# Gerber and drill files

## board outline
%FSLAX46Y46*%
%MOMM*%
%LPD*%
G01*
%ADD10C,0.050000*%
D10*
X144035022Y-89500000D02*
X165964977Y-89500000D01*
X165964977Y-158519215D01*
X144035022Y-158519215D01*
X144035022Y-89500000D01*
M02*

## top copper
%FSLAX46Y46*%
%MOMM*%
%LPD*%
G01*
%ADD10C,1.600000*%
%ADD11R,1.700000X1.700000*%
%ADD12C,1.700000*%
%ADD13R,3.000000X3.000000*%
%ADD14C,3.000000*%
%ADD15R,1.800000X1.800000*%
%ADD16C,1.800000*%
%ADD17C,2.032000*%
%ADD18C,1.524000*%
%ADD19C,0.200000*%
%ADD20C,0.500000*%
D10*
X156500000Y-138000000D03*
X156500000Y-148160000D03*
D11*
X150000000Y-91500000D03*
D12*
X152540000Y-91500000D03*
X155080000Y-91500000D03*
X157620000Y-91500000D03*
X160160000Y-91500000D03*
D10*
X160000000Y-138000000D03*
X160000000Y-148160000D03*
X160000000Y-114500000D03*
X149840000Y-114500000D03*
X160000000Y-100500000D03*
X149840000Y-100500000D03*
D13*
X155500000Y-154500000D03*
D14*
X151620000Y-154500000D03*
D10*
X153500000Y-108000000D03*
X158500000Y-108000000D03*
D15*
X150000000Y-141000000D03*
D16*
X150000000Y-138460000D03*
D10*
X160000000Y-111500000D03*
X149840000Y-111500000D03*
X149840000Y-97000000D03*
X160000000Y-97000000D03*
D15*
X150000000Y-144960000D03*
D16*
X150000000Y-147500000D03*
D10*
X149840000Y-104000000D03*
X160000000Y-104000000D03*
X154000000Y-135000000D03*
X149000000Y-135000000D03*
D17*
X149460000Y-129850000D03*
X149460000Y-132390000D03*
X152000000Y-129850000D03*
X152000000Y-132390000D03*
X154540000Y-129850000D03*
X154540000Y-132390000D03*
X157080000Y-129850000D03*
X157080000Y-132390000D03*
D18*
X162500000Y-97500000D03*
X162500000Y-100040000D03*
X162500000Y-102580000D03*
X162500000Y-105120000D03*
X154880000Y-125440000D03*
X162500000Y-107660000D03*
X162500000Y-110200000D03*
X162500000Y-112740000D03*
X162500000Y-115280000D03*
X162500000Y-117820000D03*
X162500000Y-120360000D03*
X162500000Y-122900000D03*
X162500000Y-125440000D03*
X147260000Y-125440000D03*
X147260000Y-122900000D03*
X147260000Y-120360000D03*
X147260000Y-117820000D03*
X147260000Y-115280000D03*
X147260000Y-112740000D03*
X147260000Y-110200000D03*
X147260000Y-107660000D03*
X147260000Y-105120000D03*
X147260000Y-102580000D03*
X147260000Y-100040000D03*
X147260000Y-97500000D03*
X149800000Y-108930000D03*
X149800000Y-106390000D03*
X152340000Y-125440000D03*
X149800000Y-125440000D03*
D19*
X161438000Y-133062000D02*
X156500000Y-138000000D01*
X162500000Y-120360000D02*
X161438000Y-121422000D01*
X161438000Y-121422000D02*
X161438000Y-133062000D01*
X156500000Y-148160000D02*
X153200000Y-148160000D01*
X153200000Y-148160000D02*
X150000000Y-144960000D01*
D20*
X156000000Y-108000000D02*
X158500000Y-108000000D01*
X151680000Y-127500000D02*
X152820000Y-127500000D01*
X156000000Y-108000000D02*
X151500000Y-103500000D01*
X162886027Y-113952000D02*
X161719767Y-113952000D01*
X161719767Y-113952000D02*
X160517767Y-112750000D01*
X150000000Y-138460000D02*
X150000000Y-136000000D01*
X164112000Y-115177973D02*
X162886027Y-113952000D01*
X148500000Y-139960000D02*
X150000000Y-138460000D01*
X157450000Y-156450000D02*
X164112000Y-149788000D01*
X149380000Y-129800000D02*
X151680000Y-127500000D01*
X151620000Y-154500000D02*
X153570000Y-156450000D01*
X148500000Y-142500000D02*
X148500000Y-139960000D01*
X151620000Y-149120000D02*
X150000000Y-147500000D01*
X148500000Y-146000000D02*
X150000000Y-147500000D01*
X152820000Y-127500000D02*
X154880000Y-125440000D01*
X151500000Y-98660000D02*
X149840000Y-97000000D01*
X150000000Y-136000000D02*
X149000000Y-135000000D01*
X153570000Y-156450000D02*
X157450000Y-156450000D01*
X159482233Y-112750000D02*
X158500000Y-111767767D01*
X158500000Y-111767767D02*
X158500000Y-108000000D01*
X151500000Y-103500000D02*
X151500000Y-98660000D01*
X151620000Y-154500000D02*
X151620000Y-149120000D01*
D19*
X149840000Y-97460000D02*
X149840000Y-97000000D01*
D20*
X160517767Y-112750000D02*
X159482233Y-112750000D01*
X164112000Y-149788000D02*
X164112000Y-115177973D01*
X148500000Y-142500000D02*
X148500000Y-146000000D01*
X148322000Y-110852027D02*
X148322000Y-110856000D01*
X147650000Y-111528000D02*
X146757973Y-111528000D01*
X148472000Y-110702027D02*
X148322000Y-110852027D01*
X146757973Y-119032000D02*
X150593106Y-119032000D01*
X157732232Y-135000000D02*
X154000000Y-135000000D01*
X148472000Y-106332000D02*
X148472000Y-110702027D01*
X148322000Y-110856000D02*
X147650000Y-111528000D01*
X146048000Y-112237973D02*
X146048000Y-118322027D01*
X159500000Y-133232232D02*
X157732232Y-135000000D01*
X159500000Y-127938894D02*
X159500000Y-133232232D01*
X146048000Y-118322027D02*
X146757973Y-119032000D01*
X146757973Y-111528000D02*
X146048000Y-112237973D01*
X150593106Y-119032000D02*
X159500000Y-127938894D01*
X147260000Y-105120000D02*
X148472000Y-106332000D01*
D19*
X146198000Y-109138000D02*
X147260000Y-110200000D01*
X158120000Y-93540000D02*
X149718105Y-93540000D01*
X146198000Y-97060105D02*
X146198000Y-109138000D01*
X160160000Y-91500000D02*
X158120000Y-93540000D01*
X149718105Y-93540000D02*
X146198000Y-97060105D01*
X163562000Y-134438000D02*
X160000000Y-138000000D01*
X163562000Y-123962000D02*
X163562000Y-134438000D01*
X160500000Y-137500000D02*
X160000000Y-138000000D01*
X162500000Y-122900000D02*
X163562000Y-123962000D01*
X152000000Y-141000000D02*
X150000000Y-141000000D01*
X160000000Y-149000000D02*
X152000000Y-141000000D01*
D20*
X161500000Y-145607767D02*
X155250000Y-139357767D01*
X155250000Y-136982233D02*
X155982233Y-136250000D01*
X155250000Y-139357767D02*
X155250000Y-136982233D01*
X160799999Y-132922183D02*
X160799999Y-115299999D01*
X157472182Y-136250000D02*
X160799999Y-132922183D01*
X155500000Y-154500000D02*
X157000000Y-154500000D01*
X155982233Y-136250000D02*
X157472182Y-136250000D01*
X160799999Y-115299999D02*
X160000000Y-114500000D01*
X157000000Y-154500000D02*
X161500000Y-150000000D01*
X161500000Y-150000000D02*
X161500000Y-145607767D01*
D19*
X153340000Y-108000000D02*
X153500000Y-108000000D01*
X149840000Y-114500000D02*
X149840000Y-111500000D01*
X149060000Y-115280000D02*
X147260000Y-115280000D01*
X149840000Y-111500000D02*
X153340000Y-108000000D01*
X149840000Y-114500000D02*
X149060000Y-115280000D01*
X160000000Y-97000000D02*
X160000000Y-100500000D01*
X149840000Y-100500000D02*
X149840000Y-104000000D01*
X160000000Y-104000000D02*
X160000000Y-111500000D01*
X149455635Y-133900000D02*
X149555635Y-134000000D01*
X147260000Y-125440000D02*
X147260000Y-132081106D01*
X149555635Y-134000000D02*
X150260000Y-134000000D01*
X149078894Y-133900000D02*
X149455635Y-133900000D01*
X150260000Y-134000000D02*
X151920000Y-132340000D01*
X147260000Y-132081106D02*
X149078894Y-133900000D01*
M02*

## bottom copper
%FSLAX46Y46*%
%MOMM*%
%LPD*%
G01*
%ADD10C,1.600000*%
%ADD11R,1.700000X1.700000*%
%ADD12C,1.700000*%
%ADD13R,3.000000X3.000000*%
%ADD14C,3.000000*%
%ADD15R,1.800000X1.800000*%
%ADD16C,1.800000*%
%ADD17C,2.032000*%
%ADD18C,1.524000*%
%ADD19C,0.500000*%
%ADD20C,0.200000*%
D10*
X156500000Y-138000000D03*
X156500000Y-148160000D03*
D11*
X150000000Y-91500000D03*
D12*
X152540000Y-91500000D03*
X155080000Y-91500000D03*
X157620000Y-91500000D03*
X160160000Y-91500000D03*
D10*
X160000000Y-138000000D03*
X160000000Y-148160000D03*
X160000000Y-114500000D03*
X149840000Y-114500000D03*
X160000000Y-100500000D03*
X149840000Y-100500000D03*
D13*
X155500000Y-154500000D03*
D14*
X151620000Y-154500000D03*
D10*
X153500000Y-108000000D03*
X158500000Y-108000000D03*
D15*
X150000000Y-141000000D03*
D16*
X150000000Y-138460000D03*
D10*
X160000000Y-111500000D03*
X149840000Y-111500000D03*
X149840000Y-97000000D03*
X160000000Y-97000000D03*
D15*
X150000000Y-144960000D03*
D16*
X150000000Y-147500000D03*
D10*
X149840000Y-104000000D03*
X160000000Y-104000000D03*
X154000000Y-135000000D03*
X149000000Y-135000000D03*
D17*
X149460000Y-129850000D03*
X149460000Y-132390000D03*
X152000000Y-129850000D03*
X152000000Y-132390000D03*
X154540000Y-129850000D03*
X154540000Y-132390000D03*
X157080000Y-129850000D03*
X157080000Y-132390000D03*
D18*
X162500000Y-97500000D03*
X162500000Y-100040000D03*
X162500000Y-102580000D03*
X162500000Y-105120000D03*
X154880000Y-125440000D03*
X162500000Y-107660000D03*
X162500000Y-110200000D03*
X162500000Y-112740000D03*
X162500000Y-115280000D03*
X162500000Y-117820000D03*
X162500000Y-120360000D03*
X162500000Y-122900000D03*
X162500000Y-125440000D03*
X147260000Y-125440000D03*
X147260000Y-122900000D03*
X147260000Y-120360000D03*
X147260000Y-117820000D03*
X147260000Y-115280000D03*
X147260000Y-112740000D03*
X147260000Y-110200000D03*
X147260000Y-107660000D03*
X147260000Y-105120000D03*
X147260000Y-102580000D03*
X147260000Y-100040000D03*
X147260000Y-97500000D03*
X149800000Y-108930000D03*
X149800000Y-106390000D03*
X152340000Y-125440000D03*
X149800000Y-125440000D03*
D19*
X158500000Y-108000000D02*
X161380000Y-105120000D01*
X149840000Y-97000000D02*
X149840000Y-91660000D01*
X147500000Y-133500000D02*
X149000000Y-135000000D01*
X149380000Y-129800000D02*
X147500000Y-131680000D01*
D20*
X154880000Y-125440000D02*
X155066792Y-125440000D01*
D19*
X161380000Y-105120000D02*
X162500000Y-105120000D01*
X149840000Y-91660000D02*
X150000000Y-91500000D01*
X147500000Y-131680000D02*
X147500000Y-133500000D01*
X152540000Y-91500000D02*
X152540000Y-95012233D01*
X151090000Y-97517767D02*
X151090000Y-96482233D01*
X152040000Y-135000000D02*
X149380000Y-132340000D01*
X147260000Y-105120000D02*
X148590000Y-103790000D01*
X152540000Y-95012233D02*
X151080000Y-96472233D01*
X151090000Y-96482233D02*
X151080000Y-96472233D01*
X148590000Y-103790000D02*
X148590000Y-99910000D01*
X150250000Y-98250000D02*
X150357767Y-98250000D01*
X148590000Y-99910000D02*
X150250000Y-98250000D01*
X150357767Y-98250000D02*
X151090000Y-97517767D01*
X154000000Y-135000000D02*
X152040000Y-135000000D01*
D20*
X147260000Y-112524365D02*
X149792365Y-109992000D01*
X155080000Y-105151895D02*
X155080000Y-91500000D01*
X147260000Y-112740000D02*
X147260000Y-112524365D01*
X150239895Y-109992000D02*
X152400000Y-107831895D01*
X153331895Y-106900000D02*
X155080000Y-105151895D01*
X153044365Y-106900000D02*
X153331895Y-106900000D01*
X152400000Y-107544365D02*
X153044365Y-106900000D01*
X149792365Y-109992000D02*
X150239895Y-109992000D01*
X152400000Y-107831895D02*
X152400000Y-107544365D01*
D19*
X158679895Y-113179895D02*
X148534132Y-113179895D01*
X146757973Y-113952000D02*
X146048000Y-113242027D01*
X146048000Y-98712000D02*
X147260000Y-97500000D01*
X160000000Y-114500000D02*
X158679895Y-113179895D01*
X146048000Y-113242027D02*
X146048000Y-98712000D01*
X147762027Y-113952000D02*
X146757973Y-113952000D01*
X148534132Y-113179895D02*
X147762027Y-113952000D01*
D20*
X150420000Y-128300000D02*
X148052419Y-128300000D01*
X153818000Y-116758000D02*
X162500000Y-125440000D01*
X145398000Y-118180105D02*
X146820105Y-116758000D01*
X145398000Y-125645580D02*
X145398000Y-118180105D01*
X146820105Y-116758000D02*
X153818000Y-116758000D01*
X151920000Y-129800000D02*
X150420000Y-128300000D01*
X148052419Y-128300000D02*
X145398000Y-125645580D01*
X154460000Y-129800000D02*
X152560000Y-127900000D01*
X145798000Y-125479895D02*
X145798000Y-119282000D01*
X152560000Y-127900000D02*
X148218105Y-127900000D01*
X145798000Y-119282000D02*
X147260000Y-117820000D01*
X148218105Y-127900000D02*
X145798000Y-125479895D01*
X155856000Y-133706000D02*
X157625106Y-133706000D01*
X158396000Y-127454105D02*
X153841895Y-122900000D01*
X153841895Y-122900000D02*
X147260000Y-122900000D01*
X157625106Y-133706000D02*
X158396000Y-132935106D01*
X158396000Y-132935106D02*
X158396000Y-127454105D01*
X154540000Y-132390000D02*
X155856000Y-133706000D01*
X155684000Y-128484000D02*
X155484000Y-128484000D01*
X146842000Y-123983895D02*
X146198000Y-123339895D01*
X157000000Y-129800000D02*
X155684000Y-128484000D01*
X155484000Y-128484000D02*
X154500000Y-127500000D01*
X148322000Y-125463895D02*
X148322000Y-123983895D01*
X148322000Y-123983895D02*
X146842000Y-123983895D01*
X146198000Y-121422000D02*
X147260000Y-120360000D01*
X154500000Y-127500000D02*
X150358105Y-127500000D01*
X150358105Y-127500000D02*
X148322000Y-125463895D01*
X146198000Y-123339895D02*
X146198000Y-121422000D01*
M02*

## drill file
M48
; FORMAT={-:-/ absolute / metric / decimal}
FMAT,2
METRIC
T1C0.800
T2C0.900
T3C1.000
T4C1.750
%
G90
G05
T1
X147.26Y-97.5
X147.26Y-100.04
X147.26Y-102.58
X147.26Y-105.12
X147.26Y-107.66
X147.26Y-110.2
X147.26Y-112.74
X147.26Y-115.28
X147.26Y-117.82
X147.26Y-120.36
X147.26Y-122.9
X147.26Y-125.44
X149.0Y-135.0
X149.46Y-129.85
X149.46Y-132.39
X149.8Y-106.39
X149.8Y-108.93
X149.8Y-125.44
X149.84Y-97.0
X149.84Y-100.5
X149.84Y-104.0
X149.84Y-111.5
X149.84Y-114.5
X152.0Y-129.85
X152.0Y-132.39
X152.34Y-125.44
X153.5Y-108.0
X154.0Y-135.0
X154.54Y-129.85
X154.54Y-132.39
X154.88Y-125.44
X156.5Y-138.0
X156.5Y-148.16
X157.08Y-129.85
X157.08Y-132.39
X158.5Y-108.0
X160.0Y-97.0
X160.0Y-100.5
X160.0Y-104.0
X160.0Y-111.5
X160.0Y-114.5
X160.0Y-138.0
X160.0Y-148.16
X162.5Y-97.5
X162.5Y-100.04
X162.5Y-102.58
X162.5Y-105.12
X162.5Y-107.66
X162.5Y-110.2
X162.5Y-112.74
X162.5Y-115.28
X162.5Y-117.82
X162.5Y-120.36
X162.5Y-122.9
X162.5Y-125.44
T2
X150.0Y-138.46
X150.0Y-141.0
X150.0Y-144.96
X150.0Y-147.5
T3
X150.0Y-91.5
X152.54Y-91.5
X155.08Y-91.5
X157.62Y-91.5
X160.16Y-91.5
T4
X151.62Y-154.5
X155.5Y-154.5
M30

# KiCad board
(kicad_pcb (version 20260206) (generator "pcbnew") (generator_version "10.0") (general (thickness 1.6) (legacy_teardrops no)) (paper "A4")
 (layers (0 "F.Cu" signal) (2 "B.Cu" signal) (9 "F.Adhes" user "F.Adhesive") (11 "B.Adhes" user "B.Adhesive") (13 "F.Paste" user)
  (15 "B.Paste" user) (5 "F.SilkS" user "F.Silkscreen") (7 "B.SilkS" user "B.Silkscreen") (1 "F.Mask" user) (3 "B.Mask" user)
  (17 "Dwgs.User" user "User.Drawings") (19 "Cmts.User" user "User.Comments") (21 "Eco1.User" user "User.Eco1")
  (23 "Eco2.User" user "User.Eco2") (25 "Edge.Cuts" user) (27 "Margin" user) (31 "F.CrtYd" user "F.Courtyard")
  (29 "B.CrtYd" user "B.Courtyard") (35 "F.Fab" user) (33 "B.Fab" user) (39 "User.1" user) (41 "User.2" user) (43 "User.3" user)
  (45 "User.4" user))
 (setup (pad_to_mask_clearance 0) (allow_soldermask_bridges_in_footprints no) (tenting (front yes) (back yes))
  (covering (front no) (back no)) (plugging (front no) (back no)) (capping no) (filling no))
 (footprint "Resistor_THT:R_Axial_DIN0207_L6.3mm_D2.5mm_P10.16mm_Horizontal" (layer "F.Cu") (at 156.5 138 -90)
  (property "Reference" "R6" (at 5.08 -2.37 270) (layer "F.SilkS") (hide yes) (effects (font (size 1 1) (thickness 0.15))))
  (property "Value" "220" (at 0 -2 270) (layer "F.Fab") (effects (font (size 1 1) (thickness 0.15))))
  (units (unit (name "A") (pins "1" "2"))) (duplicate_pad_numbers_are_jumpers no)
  (pad "1" thru_hole circle (at 0 0 270) (size 1.6 1.6) (drill 0.8) (layers "*.Cu" "*.Mask") (remove_unused_layers no) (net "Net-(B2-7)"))
  (pad "2" thru_hole circle (at 10.16 0 270) (size 1.6 1.6) (drill 0.8) (layers "*.Cu" "*.Mask") (remove_unused_layers no)
   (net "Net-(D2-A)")))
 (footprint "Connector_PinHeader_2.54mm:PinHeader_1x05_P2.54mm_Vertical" (layer "F.Cu") (at 150 91.5 90)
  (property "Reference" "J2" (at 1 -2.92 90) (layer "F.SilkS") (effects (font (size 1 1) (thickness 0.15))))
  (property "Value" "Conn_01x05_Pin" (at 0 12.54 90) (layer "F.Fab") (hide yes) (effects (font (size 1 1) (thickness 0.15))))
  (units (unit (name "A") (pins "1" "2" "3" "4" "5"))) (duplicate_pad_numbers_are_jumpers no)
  (pad "1" thru_hole rect (at 0 0 90) (size 1.7 1.7) (drill 1) (layers "*.Cu" "*.Mask") (remove_unused_layers no) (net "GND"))
  (pad "2" thru_hole circle (at 0 2.54 90) (size 1.7 1.7) (drill 1) (layers "*.Cu" "*.Mask") (remove_unused_layers no) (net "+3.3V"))
  (pad "3" thru_hole circle (at 0 5.08 90) (size 1.7 1.7) (drill 1) (layers "*.Cu" "*.Mask") (remove_unused_layers no) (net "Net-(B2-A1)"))
  (pad "4" thru_hole circle (at 0 7.62 90) (size 1.7 1.7) (drill 1) (layers "*.Cu" "*.Mask") (remove_unused_layers no)
   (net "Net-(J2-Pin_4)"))
  (pad "5" thru_hole circle (at 0 10.16 90) (size 1.7 1.7) (drill 1) (layers "*.Cu" "*.Mask") (remove_unused_layers no) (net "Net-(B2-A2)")))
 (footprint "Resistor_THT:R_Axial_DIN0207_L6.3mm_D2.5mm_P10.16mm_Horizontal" (layer "F.Cu") (at 160 138 -90)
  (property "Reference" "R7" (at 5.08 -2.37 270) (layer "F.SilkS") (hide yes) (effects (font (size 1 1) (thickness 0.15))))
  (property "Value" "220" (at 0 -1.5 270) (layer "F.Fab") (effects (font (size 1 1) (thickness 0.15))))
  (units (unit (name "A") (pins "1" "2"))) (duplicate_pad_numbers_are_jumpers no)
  (pad "1" thru_hole circle (at 0 0 270) (size 1.6 1.6) (drill 0.8) (layers "*.Cu" "*.Mask") (remove_unused_layers no) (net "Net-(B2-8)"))
  (pad "2" thru_hole circle (at 10.16 0 270) (size 1.6 1.6) (drill 0.8) (layers "*.Cu" "*.Mask") (remove_unused_layers no)
   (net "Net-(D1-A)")))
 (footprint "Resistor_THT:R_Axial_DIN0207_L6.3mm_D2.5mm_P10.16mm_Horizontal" (layer "F.Cu") (at 160 114.5 180)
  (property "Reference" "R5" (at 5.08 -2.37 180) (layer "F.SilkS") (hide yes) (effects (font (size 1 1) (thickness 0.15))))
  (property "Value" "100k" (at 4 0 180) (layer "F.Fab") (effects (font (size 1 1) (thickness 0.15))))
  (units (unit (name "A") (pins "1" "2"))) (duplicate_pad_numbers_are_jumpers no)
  (pad "1" thru_hole circle (at 0 0 180) (size 1.6 1.6) (drill 0.8) (layers "*.Cu" "*.Mask") (remove_unused_layers no) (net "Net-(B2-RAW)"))
  (pad "2" thru_hole circle (at 10.16 0 180) (size 1.6 1.6) (drill 0.8) (layers "*.Cu" "*.Mask") (remove_unused_layers no)
   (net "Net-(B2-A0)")))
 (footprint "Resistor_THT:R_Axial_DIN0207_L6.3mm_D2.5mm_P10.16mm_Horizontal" (layer "F.Cu") (at 160 100.5 180)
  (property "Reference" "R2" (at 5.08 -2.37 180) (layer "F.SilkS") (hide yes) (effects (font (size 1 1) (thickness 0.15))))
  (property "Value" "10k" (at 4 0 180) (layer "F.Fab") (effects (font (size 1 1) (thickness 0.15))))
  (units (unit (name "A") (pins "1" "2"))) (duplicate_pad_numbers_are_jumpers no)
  (pad "1" thru_hole circle (at 0 0 180) (size 1.6 1.6) (drill 0.8) (layers "*.Cu" "*.Mask") (remove_unused_layers no) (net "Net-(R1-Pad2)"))
  (pad "2" thru_hole circle (at 10.16 0 180) (size 1.6 1.6) (drill 0.8) (layers "*.Cu" "*.Mask") (remove_unused_layers no)
   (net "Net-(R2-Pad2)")))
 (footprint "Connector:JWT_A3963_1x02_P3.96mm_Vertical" (layer "F.Cu") (at 155.5 154.5 180)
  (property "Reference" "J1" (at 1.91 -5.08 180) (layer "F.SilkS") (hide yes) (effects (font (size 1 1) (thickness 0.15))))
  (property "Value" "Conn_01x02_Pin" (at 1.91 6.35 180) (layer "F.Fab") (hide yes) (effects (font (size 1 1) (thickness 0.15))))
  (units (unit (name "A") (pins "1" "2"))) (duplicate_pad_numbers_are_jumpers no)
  (pad "1" thru_hole rect (at 0 0 180) (size 3 3) (drill 1.75) (layers "*.Cu" "*.Mask") (remove_unused_layers no) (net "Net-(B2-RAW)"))
  (pad "2" thru_hole circle (at 3.88 0 180) (size 3 3) (drill 1.75) (layers "*.Cu" "*.Mask") (remove_unused_layers no) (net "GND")))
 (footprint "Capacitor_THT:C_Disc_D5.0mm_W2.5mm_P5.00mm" (layer "F.Cu") (at 153.5 108)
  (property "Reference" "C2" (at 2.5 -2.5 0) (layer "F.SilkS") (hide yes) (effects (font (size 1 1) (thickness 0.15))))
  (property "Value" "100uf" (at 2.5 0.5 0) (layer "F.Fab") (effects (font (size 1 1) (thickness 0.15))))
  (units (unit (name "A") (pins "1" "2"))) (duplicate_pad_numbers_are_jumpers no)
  (pad "1" thru_hole circle (at 0 0) (size 1.6 1.6) (drill 0.8) (layers "*.Cu" "*.Mask") (remove_unused_layers no) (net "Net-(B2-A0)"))
  (pad "2" thru_hole circle (at 5 0) (size 1.6 1.6) (drill 0.8) (layers "*.Cu" "*.Mask") (remove_unused_layers no) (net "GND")))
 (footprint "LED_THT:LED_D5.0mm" (layer "F.Cu") (at 150 141 90)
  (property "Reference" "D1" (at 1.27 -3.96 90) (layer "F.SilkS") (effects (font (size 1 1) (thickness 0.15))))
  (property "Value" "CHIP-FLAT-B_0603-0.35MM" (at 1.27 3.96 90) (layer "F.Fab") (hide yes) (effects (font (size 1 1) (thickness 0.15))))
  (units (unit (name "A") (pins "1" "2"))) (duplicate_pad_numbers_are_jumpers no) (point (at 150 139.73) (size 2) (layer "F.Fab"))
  (pad "1" thru_hole rect (at 0 0 90) (size 1.8 1.8) (drill 0.9) (layers "*.Cu" "*.Mask") (remove_unused_layers no) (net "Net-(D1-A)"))
  (pad "2" thru_hole circle (at 2.54 0 90) (size 1.8 1.8) (drill 0.9) (layers "*.Cu" "*.Mask") (remove_unused_layers no) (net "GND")))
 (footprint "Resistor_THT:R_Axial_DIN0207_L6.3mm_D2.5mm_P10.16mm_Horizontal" (layer "F.Cu") (at 160 111.5 180)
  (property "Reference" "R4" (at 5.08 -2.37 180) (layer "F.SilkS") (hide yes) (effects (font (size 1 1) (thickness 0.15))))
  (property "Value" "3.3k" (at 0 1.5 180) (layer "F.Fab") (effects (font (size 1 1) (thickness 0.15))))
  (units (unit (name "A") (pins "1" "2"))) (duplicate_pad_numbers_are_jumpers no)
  (pad "1" thru_hole circle (at 0 0 180) (size 1.6 1.6) (drill 0.8) (layers "*.Cu" "*.Mask") (remove_unused_layers no) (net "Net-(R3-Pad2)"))
  (pad "2" thru_hole circle (at 10.16 0 180) (size 1.6 1.6) (drill 0.8) (layers "*.Cu" "*.Mask") (remove_unused_layers no)
   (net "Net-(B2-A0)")))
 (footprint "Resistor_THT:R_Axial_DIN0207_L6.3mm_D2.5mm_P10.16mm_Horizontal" (layer "F.Cu") (at 149.84 97)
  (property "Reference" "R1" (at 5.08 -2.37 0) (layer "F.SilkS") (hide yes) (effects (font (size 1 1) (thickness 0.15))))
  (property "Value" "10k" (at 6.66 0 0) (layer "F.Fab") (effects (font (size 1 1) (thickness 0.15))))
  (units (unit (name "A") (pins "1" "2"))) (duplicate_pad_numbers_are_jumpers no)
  (pad "1" thru_hole circle (at 0 0) (size 1.6 1.6) (drill 0.8) (layers "*.Cu" "*.Mask") (remove_unused_layers no) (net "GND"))
  (pad "2" thru_hole circle (at 10.16 0) (size 1.6 1.6) (drill 0.8) (layers "*.Cu" "*.Mask") (remove_unused_layers no) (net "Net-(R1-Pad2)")))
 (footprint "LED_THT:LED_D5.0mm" (layer "F.Cu") (at 150 144.96 -90)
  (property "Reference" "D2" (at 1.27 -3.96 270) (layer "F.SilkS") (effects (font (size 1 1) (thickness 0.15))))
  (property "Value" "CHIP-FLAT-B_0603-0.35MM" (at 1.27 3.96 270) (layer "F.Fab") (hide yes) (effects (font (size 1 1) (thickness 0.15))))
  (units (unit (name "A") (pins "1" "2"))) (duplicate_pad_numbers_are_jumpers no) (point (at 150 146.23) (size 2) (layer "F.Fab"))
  (pad "1" thru_hole rect (at 0 0 270) (size 1.8 1.8) (drill 0.9) (layers "*.Cu" "*.Mask") (remove_unused_layers no) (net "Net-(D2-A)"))
  (pad "2" thru_hole circle (at 2.54 0 270) (size 1.8 1.8) (drill 0.9) (layers "*.Cu" "*.Mask") (remove_unused_layers no) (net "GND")))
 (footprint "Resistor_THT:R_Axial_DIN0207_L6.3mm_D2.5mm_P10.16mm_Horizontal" (layer "F.Cu") (at 149.84 104)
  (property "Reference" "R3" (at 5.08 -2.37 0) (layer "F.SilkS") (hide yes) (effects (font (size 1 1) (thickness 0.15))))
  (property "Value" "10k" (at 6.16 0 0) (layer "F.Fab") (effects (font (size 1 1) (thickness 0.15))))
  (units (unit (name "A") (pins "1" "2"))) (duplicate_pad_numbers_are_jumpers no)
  (pad "1" thru_hole circle (at 0 0) (size 1.6 1.6) (drill 0.8) (layers "*.Cu" "*.Mask") (remove_unused_layers no) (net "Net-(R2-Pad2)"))
  (pad "2" thru_hole circle (at 10.16 0) (size 1.6 1.6) (drill 0.8) (layers "*.Cu" "*.Mask") (remove_unused_layers no) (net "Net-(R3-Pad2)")))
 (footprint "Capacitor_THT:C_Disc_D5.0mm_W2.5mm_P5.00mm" (layer "F.Cu") (at 154 135 180)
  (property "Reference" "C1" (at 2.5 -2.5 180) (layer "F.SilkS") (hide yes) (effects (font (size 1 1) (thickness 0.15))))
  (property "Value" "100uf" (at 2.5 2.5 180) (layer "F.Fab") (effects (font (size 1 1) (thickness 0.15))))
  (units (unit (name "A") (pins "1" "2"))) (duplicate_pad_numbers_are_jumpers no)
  (pad "1" thru_hole circle (at 0 0 180) (size 1.6 1.6) (drill 0.8) (layers "*.Cu" "*.Mask") (remove_unused_layers no) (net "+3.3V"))
  (pad "2" thru_hole circle (at 5 0 180) (size 1.6 1.6) (drill 0.8) (layers "*.Cu" "*.Mask") (remove_unused_layers no) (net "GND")))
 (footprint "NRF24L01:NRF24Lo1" (layer "B.Cu") (at 155.175 142.55 -90)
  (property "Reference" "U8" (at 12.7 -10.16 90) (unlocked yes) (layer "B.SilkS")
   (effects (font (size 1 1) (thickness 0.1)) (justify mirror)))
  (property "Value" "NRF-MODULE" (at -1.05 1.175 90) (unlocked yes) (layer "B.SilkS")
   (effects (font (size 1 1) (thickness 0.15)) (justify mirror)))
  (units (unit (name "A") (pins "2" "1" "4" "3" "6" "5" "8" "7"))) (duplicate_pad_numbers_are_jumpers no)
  (pad "1" thru_hole circle (at -12.7 5.715 270) (size 2.032 2.032) (drill 0.8) (layers "*.Cu" "*.Mask") (remove_unused_layers no)
   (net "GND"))
  (pad "2" thru_hole circle (at -10.16 5.715 270) (size 2.032 2.032) (drill 0.8) (layers "*.Cu" "*.Mask") (remove_unused_layers no)
   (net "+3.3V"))
  (pad "3" thru_hole circle (at -12.7 3.175 270) (size 2.032 2.032) (drill 0.8) (layers "*.Cu" "*.Mask") (remove_unused_layers no)
   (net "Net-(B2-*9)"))
  (pad "4" thru_hole circle (at -10.16 3.175 270) (size 2.032 2.032) (drill 0.8) (layers "*.Cu" "*.Mask") (remove_unused_layers no)
   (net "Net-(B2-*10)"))
  (pad "5" thru_hole circle (at -12.7 0.635 270) (size 2.032 2.032) (drill 0.8) (layers "*.Cu" "*.Mask") (remove_unused_layers no)
   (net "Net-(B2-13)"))
  (pad "6" thru_hole circle (at -10.16 0.635 270) (size 2.032 2.032) (drill 0.8) (layers "*.Cu" "*.Mask") (remove_unused_layers no)
   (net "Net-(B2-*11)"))
  (pad "7" thru_hole circle (at -12.7 -1.905 270) (size 2.032 2.032) (drill 0.8) (layers "*.Cu" "*.Mask") (remove_unused_layers no)
   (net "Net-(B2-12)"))
  (pad "8" thru_hole circle (at -10.16 -1.905 270) (size 2.032 2.032) (drill 0.8) (layers "*.Cu" "*.Mask") (remove_unused_layers no)
   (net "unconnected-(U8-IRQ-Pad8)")))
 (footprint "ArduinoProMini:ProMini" (layer "B.Cu") (at 154.88 110.2 180)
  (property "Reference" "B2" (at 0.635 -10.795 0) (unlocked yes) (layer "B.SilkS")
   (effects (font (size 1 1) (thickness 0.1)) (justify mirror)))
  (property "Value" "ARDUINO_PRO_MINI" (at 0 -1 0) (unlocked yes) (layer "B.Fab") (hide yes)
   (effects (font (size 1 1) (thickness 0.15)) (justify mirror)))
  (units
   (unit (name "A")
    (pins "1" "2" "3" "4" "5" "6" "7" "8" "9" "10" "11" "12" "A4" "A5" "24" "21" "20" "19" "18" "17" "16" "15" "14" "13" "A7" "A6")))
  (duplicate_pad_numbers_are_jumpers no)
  (pad "1" thru_hole circle (at -7.62 12.7 180) (size 1.524 1.524) (drill 0.8) (layers "*.Cu" "*.Mask") (remove_unused_layers no)
   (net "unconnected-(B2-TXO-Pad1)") (thermal_bridge_angle 90))
  (pad "2" thru_hole circle (at -7.62 10.16 180) (size 1.524 1.524) (drill 0.8) (layers "*.Cu" "*.Mask") (remove_unused_layers no)
   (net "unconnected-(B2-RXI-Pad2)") (thermal_bridge_angle 90))
  (pad "3" thru_hole circle (at -7.62 7.62 180) (size 1.524 1.524) (drill 0.8) (layers "*.Cu" "*.Mask") (remove_unused_layers no)
   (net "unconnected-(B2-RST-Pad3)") (thermal_bridge_angle 90))
  (pad "4" thru_hole circle (at -7.62 5.08 180) (size 1.524 1.524) (drill 0.8) (layers "*.Cu" "*.Mask") (remove_unused_layers no)
   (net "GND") (thermal_bridge_angle 90))
  (pad "4" thru_hole circle (at 0 -15.24 180) (size 1.524 1.524) (drill 0.8) (layers "*.Cu" "*.Mask") (remove_unused_layers no) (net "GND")
   (thermal_bridge_angle 90))
  (pad "5" thru_hole circle (at -7.62 2.54 180) (size 1.524 1.524) (drill 0.8) (layers "*.Cu" "*.Mask") (remove_unused_layers no)
   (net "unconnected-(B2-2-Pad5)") (thermal_bridge_angle 90))
  (pad "6" thru_hole circle (at -7.62 0 180) (size 1.524 1.524) (drill 0.8) (layers "*.Cu" "*.Mask") (remove_unused_layers no)
   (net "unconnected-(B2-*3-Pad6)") (thermal_bridge_angle 90))
  (pad "7" thru_hole circle (at -7.62 -2.54 180) (size 1.524 1.524) (drill 0.8) (layers "*.Cu" "*.Mask") (remove_unused_layers no)
   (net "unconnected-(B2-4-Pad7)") (thermal_bridge_angle 90))
  (pad "8" thru_hole circle (at -7.62 -5.08 180) (size 1.524 1.524) (drill 0.8) (layers "*.Cu" "*.Mask") (remove_unused_layers no)
   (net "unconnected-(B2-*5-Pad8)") (thermal_bridge_angle 90))
  (pad "9" thru_hole circle (at -7.62 -7.62 180) (size 1.524 1.524) (drill 0.8) (layers "*.Cu" "*.Mask") (remove_unused_layers no)
   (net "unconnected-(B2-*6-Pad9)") (thermal_bridge_angle 90))
  (pad "10" thru_hole circle (at -7.62 -10.16 180) (size 1.524 1.524) (drill 0.8) (layers "*.Cu" "*.Mask") (remove_unused_layers no)
   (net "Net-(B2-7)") (thermal_bridge_angle 90))
  (pad "11" thru_hole circle (at -7.62 -12.7 180) (size 1.524 1.524) (drill 0.8) (layers "*.Cu" "*.Mask") (remove_unused_layers no)
   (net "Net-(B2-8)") (thermal_bridge_angle 90))
  (pad "12" thru_hole circle (at -7.62 -15.24 180) (size 1.524 1.524) (drill 0.8) (layers "*.Cu" "*.Mask") (remove_unused_layers no)
   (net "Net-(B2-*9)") (thermal_bridge_angle 90))
  (pad "13" thru_hole circle (at 7.62 -15.24 180) (size 1.524 1.524) (drill 0.8) (layers "*.Cu" "*.Mask") (remove_unused_layers no)
   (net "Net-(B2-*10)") (thermal_bridge_angle 90))
  (pad "14" thru_hole circle (at 7.62 -12.7 180) (size 1.524 1.524) (drill 0.8) (layers "*.Cu" "*.Mask") (remove_unused_layers no)
   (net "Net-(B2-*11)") (thermal_bridge_angle 90))
  (pad "15" thru_hole circle (at 7.62 -10.16 180) (size 1.524 1.524) (drill 0.8) (layers "*.Cu" "*.Mask") (remove_unused_layers no)
   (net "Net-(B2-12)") (thermal_bridge_angle 90))
  (pad "16" thru_hole circle (at 7.62 -7.62 180) (size 1.524 1.524) (drill 0.8) (layers "*.Cu" "*.Mask") (remove_unused_layers no)
   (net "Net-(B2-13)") (thermal_bridge_angle 90))
  (pad "17" thru_hole circle (at 7.62 -5.08 180) (size 1.524 1.524) (drill 0.8) (layers "*.Cu" "*.Mask") (remove_unused_layers no)
   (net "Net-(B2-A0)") (thermal_bridge_angle 90))
  (pad "18" thru_hole circle (at 7.62 -2.54 180) (size 1.524 1.524) (drill 0.8) (layers "*.Cu" "*.Mask") (remove_unused_layers no)
   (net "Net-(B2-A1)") (thermal_bridge_angle 90))
  (pad "19" thru_hole circle (at 7.62 0 180) (size 1.524 1.524) (drill 0.8) (layers "*.Cu" "*.Mask") (remove_unused_layers no)
   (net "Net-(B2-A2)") (thermal_bridge_angle 90))
  (pad "20" thru_hole circle (at 7.62 2.54 180) (size 1.524 1.524) (drill 0.8) (layers "*.Cu" "*.Mask") (remove_unused_layers no)
   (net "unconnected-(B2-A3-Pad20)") (thermal_bridge_angle 90))
  (pad "21" thru_hole circle (at 7.62 5.08 180) (size 1.524 1.524) (drill 0.8) (layers "*.Cu" "*.Mask") (remove_unused_layers no)
   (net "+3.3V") (thermal_bridge_angle 90))
  (pad "22" thru_hole circle (at 7.62 7.62 180) (size 1.524 1.524) (drill 0.8) (layers "*.Cu" "*.Mask") (remove_unused_layers no)
   (thermal_bridge_angle 90))
  (pad "23" thru_hole circle (at 7.62 10.16 180) (size 1.524 1.524) (drill 0.8) (layers "*.Cu" "*.Mask") (remove_unused_layers no)
   (thermal_bridge_angle 90))
  (pad "24" thru_hole circle (at 7.62 12.7 180) (size 1.524 1.524) (drill 0.8) (layers "*.Cu" "*.Mask") (remove_unused_layers no)
   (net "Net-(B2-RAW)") (thermal_bridge_angle 90))
  (pad "A4" thru_hole circle (at 5.08 1.27 180) (size 1.524 1.524) (drill 0.8) (layers "*.Cu" "*.Mask") (remove_unused_layers no)
   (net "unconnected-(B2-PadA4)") (thermal_bridge_angle 90))
  (pad "A5" thru_hole circle (at 5.08 3.81 180) (size 1.524 1.524) (drill 0.8) (layers "*.Cu" "*.Mask") (remove_unused_layers no)
   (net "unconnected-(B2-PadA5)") (thermal_bridge_angle 90))
  (pad "A6" thru_hole circle (at 2.54 -15.24 180) (size 1.524 1.524) (drill 0.8) (layers "*.Cu" "*.Mask") (remove_unused_layers no)
   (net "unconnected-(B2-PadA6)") (thermal_bridge_angle 90))
  (pad "A7" thru_hole circle (at 5.08 -15.24 180) (size 1.524 1.524) (drill 0.8) (layers "*.Cu" "*.Mask") (remove_unused_layers no)
   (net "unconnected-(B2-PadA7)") (thermal_bridge_angle 90)))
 (gr_rect (start 144.035022 89.5) (end 165.964977 158.519215) (stroke (width 0.05) (type default)) (fill no) (layer "Edge.Cuts"))
 (segment (start 161.438 133.062) (end 156.5 138) (width 0.2) (layer "F.Cu") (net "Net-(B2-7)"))
 (segment (start 162.5 120.36) (end 161.438 121.422) (width 0.2) (layer "F.Cu") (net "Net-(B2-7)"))
 (segment (start 161.438 121.422) (end 161.438 133.062) (width 0.2) (layer "F.Cu") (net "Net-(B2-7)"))
 (segment (start 156.5 148.16) (end 153.2 148.16) (width 0.2) (layer "F.Cu") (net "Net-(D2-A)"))
 (segment (start 153.2 148.16) (end 150 144.96) (width 0.2) (layer "F.Cu") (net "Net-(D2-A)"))
 (segment (start 156 108) (end 158.5 108) (width 0.5) (layer "F.Cu") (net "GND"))
 (segment (start 151.68 127.5) (end 152.82 127.5) (width 0.5) (layer "F.Cu") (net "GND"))
 (segment (start 156 108) (end 151.5 103.5) (width 0.5) (layer "F.Cu") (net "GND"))
 (segment (start 162.886027 113.952) (end 161.719767 113.952) (width 0.5) (layer "F.Cu") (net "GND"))
 (segment (start 161.719767 113.952) (end 160.517767 112.75) (width 0.5) (layer "F.Cu") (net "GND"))
 (segment (start 150 138.46) (end 150 136) (width 0.5) (layer "F.Cu") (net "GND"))
 (segment (start 164.112 115.177973) (end 162.886027 113.952) (width 0.5) (layer "F.Cu") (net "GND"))
 (segment (start 148.5 139.96) (end 150 138.46) (width 0.5) (layer "F.Cu") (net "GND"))
 (segment (start 157.45 156.45) (end 164.112 149.788) (width 0.5) (layer "F.Cu") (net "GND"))
 (segment (start 149.38 129.8) (end 151.68 127.5) (width 0.5) (layer "F.Cu") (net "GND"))
 (segment (start 151.62 154.5) (end 153.57 156.45) (width 0.5) (layer "F.Cu") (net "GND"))
 (segment (start 148.5 142.5) (end 148.5 139.96) (width 0.5) (layer "F.Cu") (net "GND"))
 (segment (start 151.62 149.12) (end 150 147.5) (width 0.5) (layer "F.Cu") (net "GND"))
 (segment (start 148.5 146) (end 150 147.5) (width 0.5) (layer "F.Cu") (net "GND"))
 (segment (start 152.82 127.5) (end 154.88 125.44) (width 0.5) (layer "F.Cu") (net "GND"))
 (segment (start 151.5 98.66) (end 149.84 97) (width 0.5) (layer "F.Cu") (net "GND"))
 (segment (start 150 136) (end 149 135) (width 0.5) (layer "F.Cu") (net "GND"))
 (segment (start 153.57 156.45) (end 157.45 156.45) (width 0.5) (layer "F.Cu") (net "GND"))
 (segment (start 159.482233 112.75) (end 158.5 111.767767) (width 0.5) (layer "F.Cu") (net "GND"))
 (segment (start 158.5 111.767767) (end 158.5 108) (width 0.5) (layer "F.Cu") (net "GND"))
 (segment (start 151.5 103.5) (end 151.5 98.66) (width 0.5) (layer "F.Cu") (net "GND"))
 (segment (start 151.62 154.5) (end 151.62 149.12) (width 0.5) (layer "F.Cu") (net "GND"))
 (segment (start 149.84 97.46) (end 149.84 97) (width 0.2) (layer "F.Cu") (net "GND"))
 (segment (start 160.517767 112.75) (end 159.482233 112.75) (width 0.5) (layer "F.Cu") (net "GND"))
 (segment (start 164.112 149.788) (end 164.112 115.177973) (width 0.5) (layer "F.Cu") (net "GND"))
 (segment (start 148.5 142.5) (end 148.5 146) (width 0.5) (layer "F.Cu") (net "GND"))
 (segment (start 158.5 108) (end 161.38 105.12) (width 0.5) (layer "B.Cu") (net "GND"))
 (segment (start 149.84 97) (end 149.84 91.66) (width 0.5) (layer "B.Cu") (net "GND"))
 (segment (start 147.5 133.5) (end 149 135) (width 0.5) (layer "B.Cu") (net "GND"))
 (segment (start 149.38 129.8) (end 147.5 131.68) (width 0.5) (layer "B.Cu") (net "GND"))
 (segment (start 154.88 125.44) (end 155.066792 125.44) (width 0.2) (layer "B.Cu") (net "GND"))
 (segment (start 161.38 105.12) (end 162.5 105.12) (width 0.5) (layer "B.Cu") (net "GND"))
 (segment (start 149.84 91.66) (end 150 91.5) (width 0.5) (layer "B.Cu") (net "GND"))
 (segment (start 147.5 131.68) (end 147.5 133.5) (width 0.5) (layer "B.Cu") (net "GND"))
 (segment (start 148.322 110.852027) (end 148.322 110.856) (width 0.5) (layer "F.Cu") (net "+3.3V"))
 (segment (start 147.65 111.528) (end 146.757973 111.528) (width 0.5) (layer "F.Cu") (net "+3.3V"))
 (segment (start 148.472 110.702027) (end 148.322 110.852027) (width 0.5) (layer "F.Cu") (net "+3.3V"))
 (segment (start 146.757973 119.032) (end 150.593106 119.032) (width 0.5) (layer "F.Cu") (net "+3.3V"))
 (segment (start 157.732232 135) (end 154 135) (width 0.5) (layer "F.Cu") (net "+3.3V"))
 (segment (start 148.472 106.332) (end 148.472 110.702027) (width 0.5) (layer "F.Cu") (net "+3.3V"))
 (segment (start 148.322 110.856) (end 147.65 111.528) (width 0.5) (layer "F.Cu") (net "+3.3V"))
 (segment (start 146.048 112.237973) (end 146.048 118.322027) (width 0.5) (layer "F.Cu") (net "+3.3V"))
 (segment (start 159.5 133.232232) (end 157.732232 135) (width 0.5) (layer "F.Cu") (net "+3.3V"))
 (segment (start 159.5 127.938894) (end 159.5 133.232232) (width 0.5) (layer "F.Cu") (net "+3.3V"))
 (segment (start 146.048 118.322027) (end 146.757973 119.032) (width 0.5) (layer "F.Cu") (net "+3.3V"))
 (segment (start 146.757973 111.528) (end 146.048 112.237973) (width 0.5) (layer "F.Cu") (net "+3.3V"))
 (segment (start 150.593106 119.032) (end 159.5 127.938894) (width 0.5) (layer "F.Cu") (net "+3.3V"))
 (segment (start 147.26 105.12) (end 148.472 106.332) (width 0.5) (layer "F.Cu") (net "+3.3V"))
 (segment (start 152.54 91.5) (end 152.54 95.012233) (width 0.5) (layer "B.Cu") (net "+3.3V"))
 (segment (start 151.09 97.517767) (end 151.09 96.482233) (width 0.5) (layer "B.Cu") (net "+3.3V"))
 (segment (start 152.04 135) (end 149.38 132.34) (width 0.5) (layer "B.Cu") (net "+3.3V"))
 (segment (start 147.26 105.12) (end 148.59 103.79) (width 0.5) (layer "B.Cu") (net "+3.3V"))
 (segment (start 152.54 95.012233) (end 151.08 96.472233) (width 0.5) (layer "B.Cu") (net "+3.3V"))
 (segment (start 151.09 96.482233) (end 151.08 96.472233) (width 0.5) (layer "B.Cu") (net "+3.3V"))
 (segment (start 148.59 103.79) (end 148.59 99.91) (width 0.5) (layer "B.Cu") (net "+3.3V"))
 (segment (start 150.25 98.25) (end 150.357767 98.25) (width 0.5) (layer "B.Cu") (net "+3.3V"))
 (segment (start 148.59 99.91) (end 150.25 98.25) (width 0.5) (layer "B.Cu") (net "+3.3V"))
 (segment (start 150.357767 98.25) (end 151.09 97.517767) (width 0.5) (layer "B.Cu") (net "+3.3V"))
 (segment (start 154 135) (end 152.04 135) (width 0.5) (layer "B.Cu") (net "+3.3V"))
 (segment (start 147.26 112.524365) (end 149.792365 109.992) (width 0.2) (layer "B.Cu") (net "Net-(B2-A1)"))
 (segment (start 155.08 105.151895) (end 155.08 91.5) (width 0.2) (layer "B.Cu") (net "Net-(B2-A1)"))
 (segment (start 147.26 112.74) (end 147.26 112.524365) (width 0.2) (layer "B.Cu") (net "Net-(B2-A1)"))
 (segment (start 150.239895 109.992) (end 152.4 107.831895) (width 0.2) (layer "B.Cu") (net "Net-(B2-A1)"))
 (segment (start 153.331895 106.9) (end 155.08 105.151895) (width 0.2) (layer "B.Cu") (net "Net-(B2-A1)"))
 (segment (start 153.044365 106.9) (end 153.331895 106.9) (width 0.2) (layer "B.Cu") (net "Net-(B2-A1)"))
 (segment (start 152.4 107.544365) (end 153.044365 106.9) (width 0.2) (layer "B.Cu") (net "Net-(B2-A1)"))
 (segment (start 149.792365 109.992) (end 150.239895 109.992) (width 0.2) (layer "B.Cu") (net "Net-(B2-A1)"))
 (segment (start 152.4 107.831895) (end 152.4 107.544365) (width 0.2) (layer "B.Cu") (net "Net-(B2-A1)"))
 (segment (start 146.198 109.138) (end 147.26 110.2) (width 0.2) (layer "F.Cu") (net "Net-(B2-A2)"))
 (segment (start 158.12 93.54) (end 149.718105 93.54) (width 0.2) (layer "F.Cu") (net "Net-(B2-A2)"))
 (segment (start 146.198 97.060105) (end 146.198 109.138) (width 0.2) (layer "F.Cu") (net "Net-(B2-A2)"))
 (segment (start 160.16 91.5) (end 158.12 93.54) (width 0.2) (layer "F.Cu") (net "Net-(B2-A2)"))
 (segment (start 149.718105 93.54) (end 146.198 97.060105) (width 0.2) (layer "F.Cu") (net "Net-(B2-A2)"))
 (segment (start 163.562 134.438) (end 160 138) (width 0.2) (layer "F.Cu") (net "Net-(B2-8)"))
 (segment (start 163.562 123.962) (end 163.562 134.438) (width 0.2) (layer "F.Cu") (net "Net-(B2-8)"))
 (segment (start 160.5 137.5) (end 160 138) (width 0.2) (layer "F.Cu") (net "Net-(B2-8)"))
 (segment (start 162.5 122.9) (end 163.562 123.962) (width 0.2) (layer "F.Cu") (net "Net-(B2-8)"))
 (segment (start 152 141) (end 150 141) (width 0.2) (layer "F.Cu") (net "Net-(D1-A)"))
 (segment (start 160 149) (end 152 141) (width 0.2) (layer "F.Cu") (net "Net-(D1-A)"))
 (segment (start 161.5 145.607767) (end 155.25 139.357767) (width 0.5) (layer "F.Cu") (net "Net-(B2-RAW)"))
 (segment (start 155.25 136.982233) (end 155.982233 136.25) (width 0.5) (layer "F.Cu") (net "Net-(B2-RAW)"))
 (segment (start 155.25 139.357767) (end 155.25 136.982233) (width 0.5) (layer "F.Cu") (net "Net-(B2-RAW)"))
 (segment (start 160.799999 132.922183) (end 160.799999 115.299999) (width 0.5) (layer "F.Cu") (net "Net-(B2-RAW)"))
 (segment (start 157.472182 136.25) (end 160.799999 132.922183) (width 0.5) (layer "F.Cu") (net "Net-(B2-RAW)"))
 (segment (start 155.5 154.5) (end 157 154.5) (width 0.5) (layer "F.Cu") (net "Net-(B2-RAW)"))
 (segment (start 155.982233 136.25) (end 157.472182 136.25) (width 0.5) (layer "F.Cu") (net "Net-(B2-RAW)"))
 (segment (start 160.799999 115.299999) (end 160 114.5) (width 0.5) (layer "F.Cu") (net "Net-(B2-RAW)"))
 (segment (start 157 154.5) (end 161.5 150) (width 0.5) (layer "F.Cu") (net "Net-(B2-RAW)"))
 (segment (start 161.5 150) (end 161.5 145.607767) (width 0.5) (layer "F.Cu") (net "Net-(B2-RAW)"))
 (segment (start 158.679895 113.179895) (end 148.534132 113.179895) (width 0.5) (layer "B.Cu") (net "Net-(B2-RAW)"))
 (segment (start 146.757973 113.952) (end 146.048 113.242027) (width 0.5) (layer "B.Cu") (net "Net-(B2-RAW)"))
 (segment (start 146.048 98.712) (end 147.26 97.5) (width 0.5) (layer "B.Cu") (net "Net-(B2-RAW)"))
 (segment (start 160 114.5) (end 158.679895 113.179895) (width 0.5) (layer "B.Cu") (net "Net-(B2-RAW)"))
 (segment (start 146.048 113.242027) (end 146.048 98.712) (width 0.5) (layer "B.Cu") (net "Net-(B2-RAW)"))
 (segment (start 147.762027 113.952) (end 146.757973 113.952) (width 0.5) (layer "B.Cu") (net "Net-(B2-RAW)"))
 (segment (start 148.534132 113.179895) (end 147.762027 113.952) (width 0.5) (layer "B.Cu") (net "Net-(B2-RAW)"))
 (segment (start 153.34 108) (end 153.5 108) (width 0.2) (layer "F.Cu") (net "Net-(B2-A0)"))
 (segment (start 149.84 114.5) (end 149.84 111.5) (width 0.2) (layer "F.Cu") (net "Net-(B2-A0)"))
 (segment (start 149.06 115.28) (end 147.26 115.28) (width 0.2) (layer "F.Cu") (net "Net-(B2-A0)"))
 (segment (start 149.84 111.5) (end 153.34 108) (width 0.2) (layer "F.Cu") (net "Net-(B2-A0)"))
 (segment (start 149.84 114.5) (end 149.06 115.28) (width 0.2) (layer "F.Cu") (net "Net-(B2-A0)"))
 (segment (start 160 97) (end 160 100.5) (width 0.2) (layer "F.Cu") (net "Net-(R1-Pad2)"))
 (segment (start 149.84 100.5) (end 149.84 104) (width 0.2) (layer "F.Cu") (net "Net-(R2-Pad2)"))
 (segment (start 160 104) (end 160 111.5) (width 0.2) (layer "F.Cu") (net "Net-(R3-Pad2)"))
 (segment (start 150.42 128.3) (end 148.052419 128.3) (width 0.2) (layer "B.Cu") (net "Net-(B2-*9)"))
 (segment (start 153.818 116.758) (end 162.5 125.44) (width 0.2) (layer "B.Cu") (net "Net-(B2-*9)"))
 (segment (start 145.398 118.180105) (end 146.820105 116.758) (width 0.2) (layer "B.Cu") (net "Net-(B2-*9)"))
 (segment (start 145.398 125.64558) (end 145.398 118.180105) (width 0.2) (layer "B.Cu") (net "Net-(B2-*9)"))
 (segment (start 146.820105 116.758) (end 153.818 116.758) (width 0.2) (layer "B.Cu") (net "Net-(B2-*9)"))
 (segment (start 151.92 129.8) (end 150.42 128.3) (width 0.2) (layer "B.Cu") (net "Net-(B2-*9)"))
 (segment (start 148.052419 128.3) (end 145.398 125.64558) (width 0.2) (layer "B.Cu") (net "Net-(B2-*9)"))
 (segment (start 149.455635 133.9) (end 149.555635 134) (width 0.2) (layer "F.Cu") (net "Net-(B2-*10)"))
 (segment (start 147.26 125.44) (end 147.26 132.081106) (width 0.2) (layer "F.Cu") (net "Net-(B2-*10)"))
 (segment (start 149.555635 134) (end 150.26 134) (width 0.2) (layer "F.Cu") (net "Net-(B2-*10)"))
 (segment (start 149.078894 133.9) (end 149.455635 133.9) (width 0.2) (layer "F.Cu") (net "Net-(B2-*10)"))
 (segment (start 150.26 134) (end 151.92 132.34) (width 0.2) (layer "F.Cu") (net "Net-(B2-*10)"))
 (segment (start 147.26 132.081106) (end 149.078894 133.9) (width 0.2) (layer "F.Cu") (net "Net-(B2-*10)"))
 (segment (start 154.46 129.8) (end 152.56 127.9) (width 0.2) (layer "B.Cu") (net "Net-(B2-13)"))
 (segment (start 145.798 125.479895) (end 145.798 119.282) (width 0.2) (layer "B.Cu") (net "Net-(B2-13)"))
 (segment (start 152.56 127.9) (end 148.218105 127.9) (width 0.2) (layer "B.Cu") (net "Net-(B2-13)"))
 (segment (start 145.798 119.282) (end 147.26 117.82) (width 0.2) (layer "B.Cu") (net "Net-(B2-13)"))
 (segment (start 148.218105 127.9) (end 145.798 125.479895) (width 0.2) (layer "B.Cu") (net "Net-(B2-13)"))
 (segment (start 155.856 133.706) (end 157.625106 133.706) (width 0.2) (layer "B.Cu") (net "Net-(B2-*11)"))
 (segment (start 158.396 127.454105) (end 153.841895 122.9) (width 0.2) (layer "B.Cu") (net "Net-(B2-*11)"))
 (segment (start 153.841895 122.9) (end 147.26 122.9) (width 0.2) (layer "B.Cu") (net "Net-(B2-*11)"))
 (segment (start 157.625106 133.706) (end 158.396 132.935106) (width 0.2) (layer "B.Cu") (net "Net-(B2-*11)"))
 (segment (start 158.396 132.935106) (end 158.396 127.454105) (width 0.2) (layer "B.Cu") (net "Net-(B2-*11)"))
 (segment (start 154.54 132.39) (end 155.856 133.706) (width 0.2) (layer "B.Cu") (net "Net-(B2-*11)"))
 (segment (start 155.684 128.484) (end 155.484 128.484) (width 0.2) (layer "B.Cu") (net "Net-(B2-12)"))
 (segment (start 146.842 123.983895) (end 146.198 123.339895) (width 0.2) (layer "B.Cu") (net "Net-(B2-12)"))
 (segment (start 157 129.8) (end 155.684 128.484) (width 0.2) (layer "B.Cu") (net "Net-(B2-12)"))
 (segment (start 155.484 128.484) (end 154.5 127.5) (width 0.2) (layer "B.Cu") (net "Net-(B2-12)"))
 (segment (start 148.322 125.463895) (end 148.322 123.983895) (width 0.2) (layer "B.Cu") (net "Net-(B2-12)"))
 (segment (start 148.322 123.983895) (end 146.842 123.983895) (width 0.2) (layer "B.Cu") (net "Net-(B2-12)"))
 (segment (start 146.198 121.422) (end 147.26 120.36) (width 0.2) (layer "B.Cu") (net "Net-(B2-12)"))
 (segment (start 154.5 127.5) (end 150.358105 127.5) (width 0.2) (layer "B.Cu") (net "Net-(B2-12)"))
 (segment (start 150.358105 127.5) (end 148.322 125.463895) (width 0.2) (layer "B.Cu") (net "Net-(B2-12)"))
 (segment (start 146.198 123.339895) (end 146.198 121.422) (width 0.2) (layer "B.Cu") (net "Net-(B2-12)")))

